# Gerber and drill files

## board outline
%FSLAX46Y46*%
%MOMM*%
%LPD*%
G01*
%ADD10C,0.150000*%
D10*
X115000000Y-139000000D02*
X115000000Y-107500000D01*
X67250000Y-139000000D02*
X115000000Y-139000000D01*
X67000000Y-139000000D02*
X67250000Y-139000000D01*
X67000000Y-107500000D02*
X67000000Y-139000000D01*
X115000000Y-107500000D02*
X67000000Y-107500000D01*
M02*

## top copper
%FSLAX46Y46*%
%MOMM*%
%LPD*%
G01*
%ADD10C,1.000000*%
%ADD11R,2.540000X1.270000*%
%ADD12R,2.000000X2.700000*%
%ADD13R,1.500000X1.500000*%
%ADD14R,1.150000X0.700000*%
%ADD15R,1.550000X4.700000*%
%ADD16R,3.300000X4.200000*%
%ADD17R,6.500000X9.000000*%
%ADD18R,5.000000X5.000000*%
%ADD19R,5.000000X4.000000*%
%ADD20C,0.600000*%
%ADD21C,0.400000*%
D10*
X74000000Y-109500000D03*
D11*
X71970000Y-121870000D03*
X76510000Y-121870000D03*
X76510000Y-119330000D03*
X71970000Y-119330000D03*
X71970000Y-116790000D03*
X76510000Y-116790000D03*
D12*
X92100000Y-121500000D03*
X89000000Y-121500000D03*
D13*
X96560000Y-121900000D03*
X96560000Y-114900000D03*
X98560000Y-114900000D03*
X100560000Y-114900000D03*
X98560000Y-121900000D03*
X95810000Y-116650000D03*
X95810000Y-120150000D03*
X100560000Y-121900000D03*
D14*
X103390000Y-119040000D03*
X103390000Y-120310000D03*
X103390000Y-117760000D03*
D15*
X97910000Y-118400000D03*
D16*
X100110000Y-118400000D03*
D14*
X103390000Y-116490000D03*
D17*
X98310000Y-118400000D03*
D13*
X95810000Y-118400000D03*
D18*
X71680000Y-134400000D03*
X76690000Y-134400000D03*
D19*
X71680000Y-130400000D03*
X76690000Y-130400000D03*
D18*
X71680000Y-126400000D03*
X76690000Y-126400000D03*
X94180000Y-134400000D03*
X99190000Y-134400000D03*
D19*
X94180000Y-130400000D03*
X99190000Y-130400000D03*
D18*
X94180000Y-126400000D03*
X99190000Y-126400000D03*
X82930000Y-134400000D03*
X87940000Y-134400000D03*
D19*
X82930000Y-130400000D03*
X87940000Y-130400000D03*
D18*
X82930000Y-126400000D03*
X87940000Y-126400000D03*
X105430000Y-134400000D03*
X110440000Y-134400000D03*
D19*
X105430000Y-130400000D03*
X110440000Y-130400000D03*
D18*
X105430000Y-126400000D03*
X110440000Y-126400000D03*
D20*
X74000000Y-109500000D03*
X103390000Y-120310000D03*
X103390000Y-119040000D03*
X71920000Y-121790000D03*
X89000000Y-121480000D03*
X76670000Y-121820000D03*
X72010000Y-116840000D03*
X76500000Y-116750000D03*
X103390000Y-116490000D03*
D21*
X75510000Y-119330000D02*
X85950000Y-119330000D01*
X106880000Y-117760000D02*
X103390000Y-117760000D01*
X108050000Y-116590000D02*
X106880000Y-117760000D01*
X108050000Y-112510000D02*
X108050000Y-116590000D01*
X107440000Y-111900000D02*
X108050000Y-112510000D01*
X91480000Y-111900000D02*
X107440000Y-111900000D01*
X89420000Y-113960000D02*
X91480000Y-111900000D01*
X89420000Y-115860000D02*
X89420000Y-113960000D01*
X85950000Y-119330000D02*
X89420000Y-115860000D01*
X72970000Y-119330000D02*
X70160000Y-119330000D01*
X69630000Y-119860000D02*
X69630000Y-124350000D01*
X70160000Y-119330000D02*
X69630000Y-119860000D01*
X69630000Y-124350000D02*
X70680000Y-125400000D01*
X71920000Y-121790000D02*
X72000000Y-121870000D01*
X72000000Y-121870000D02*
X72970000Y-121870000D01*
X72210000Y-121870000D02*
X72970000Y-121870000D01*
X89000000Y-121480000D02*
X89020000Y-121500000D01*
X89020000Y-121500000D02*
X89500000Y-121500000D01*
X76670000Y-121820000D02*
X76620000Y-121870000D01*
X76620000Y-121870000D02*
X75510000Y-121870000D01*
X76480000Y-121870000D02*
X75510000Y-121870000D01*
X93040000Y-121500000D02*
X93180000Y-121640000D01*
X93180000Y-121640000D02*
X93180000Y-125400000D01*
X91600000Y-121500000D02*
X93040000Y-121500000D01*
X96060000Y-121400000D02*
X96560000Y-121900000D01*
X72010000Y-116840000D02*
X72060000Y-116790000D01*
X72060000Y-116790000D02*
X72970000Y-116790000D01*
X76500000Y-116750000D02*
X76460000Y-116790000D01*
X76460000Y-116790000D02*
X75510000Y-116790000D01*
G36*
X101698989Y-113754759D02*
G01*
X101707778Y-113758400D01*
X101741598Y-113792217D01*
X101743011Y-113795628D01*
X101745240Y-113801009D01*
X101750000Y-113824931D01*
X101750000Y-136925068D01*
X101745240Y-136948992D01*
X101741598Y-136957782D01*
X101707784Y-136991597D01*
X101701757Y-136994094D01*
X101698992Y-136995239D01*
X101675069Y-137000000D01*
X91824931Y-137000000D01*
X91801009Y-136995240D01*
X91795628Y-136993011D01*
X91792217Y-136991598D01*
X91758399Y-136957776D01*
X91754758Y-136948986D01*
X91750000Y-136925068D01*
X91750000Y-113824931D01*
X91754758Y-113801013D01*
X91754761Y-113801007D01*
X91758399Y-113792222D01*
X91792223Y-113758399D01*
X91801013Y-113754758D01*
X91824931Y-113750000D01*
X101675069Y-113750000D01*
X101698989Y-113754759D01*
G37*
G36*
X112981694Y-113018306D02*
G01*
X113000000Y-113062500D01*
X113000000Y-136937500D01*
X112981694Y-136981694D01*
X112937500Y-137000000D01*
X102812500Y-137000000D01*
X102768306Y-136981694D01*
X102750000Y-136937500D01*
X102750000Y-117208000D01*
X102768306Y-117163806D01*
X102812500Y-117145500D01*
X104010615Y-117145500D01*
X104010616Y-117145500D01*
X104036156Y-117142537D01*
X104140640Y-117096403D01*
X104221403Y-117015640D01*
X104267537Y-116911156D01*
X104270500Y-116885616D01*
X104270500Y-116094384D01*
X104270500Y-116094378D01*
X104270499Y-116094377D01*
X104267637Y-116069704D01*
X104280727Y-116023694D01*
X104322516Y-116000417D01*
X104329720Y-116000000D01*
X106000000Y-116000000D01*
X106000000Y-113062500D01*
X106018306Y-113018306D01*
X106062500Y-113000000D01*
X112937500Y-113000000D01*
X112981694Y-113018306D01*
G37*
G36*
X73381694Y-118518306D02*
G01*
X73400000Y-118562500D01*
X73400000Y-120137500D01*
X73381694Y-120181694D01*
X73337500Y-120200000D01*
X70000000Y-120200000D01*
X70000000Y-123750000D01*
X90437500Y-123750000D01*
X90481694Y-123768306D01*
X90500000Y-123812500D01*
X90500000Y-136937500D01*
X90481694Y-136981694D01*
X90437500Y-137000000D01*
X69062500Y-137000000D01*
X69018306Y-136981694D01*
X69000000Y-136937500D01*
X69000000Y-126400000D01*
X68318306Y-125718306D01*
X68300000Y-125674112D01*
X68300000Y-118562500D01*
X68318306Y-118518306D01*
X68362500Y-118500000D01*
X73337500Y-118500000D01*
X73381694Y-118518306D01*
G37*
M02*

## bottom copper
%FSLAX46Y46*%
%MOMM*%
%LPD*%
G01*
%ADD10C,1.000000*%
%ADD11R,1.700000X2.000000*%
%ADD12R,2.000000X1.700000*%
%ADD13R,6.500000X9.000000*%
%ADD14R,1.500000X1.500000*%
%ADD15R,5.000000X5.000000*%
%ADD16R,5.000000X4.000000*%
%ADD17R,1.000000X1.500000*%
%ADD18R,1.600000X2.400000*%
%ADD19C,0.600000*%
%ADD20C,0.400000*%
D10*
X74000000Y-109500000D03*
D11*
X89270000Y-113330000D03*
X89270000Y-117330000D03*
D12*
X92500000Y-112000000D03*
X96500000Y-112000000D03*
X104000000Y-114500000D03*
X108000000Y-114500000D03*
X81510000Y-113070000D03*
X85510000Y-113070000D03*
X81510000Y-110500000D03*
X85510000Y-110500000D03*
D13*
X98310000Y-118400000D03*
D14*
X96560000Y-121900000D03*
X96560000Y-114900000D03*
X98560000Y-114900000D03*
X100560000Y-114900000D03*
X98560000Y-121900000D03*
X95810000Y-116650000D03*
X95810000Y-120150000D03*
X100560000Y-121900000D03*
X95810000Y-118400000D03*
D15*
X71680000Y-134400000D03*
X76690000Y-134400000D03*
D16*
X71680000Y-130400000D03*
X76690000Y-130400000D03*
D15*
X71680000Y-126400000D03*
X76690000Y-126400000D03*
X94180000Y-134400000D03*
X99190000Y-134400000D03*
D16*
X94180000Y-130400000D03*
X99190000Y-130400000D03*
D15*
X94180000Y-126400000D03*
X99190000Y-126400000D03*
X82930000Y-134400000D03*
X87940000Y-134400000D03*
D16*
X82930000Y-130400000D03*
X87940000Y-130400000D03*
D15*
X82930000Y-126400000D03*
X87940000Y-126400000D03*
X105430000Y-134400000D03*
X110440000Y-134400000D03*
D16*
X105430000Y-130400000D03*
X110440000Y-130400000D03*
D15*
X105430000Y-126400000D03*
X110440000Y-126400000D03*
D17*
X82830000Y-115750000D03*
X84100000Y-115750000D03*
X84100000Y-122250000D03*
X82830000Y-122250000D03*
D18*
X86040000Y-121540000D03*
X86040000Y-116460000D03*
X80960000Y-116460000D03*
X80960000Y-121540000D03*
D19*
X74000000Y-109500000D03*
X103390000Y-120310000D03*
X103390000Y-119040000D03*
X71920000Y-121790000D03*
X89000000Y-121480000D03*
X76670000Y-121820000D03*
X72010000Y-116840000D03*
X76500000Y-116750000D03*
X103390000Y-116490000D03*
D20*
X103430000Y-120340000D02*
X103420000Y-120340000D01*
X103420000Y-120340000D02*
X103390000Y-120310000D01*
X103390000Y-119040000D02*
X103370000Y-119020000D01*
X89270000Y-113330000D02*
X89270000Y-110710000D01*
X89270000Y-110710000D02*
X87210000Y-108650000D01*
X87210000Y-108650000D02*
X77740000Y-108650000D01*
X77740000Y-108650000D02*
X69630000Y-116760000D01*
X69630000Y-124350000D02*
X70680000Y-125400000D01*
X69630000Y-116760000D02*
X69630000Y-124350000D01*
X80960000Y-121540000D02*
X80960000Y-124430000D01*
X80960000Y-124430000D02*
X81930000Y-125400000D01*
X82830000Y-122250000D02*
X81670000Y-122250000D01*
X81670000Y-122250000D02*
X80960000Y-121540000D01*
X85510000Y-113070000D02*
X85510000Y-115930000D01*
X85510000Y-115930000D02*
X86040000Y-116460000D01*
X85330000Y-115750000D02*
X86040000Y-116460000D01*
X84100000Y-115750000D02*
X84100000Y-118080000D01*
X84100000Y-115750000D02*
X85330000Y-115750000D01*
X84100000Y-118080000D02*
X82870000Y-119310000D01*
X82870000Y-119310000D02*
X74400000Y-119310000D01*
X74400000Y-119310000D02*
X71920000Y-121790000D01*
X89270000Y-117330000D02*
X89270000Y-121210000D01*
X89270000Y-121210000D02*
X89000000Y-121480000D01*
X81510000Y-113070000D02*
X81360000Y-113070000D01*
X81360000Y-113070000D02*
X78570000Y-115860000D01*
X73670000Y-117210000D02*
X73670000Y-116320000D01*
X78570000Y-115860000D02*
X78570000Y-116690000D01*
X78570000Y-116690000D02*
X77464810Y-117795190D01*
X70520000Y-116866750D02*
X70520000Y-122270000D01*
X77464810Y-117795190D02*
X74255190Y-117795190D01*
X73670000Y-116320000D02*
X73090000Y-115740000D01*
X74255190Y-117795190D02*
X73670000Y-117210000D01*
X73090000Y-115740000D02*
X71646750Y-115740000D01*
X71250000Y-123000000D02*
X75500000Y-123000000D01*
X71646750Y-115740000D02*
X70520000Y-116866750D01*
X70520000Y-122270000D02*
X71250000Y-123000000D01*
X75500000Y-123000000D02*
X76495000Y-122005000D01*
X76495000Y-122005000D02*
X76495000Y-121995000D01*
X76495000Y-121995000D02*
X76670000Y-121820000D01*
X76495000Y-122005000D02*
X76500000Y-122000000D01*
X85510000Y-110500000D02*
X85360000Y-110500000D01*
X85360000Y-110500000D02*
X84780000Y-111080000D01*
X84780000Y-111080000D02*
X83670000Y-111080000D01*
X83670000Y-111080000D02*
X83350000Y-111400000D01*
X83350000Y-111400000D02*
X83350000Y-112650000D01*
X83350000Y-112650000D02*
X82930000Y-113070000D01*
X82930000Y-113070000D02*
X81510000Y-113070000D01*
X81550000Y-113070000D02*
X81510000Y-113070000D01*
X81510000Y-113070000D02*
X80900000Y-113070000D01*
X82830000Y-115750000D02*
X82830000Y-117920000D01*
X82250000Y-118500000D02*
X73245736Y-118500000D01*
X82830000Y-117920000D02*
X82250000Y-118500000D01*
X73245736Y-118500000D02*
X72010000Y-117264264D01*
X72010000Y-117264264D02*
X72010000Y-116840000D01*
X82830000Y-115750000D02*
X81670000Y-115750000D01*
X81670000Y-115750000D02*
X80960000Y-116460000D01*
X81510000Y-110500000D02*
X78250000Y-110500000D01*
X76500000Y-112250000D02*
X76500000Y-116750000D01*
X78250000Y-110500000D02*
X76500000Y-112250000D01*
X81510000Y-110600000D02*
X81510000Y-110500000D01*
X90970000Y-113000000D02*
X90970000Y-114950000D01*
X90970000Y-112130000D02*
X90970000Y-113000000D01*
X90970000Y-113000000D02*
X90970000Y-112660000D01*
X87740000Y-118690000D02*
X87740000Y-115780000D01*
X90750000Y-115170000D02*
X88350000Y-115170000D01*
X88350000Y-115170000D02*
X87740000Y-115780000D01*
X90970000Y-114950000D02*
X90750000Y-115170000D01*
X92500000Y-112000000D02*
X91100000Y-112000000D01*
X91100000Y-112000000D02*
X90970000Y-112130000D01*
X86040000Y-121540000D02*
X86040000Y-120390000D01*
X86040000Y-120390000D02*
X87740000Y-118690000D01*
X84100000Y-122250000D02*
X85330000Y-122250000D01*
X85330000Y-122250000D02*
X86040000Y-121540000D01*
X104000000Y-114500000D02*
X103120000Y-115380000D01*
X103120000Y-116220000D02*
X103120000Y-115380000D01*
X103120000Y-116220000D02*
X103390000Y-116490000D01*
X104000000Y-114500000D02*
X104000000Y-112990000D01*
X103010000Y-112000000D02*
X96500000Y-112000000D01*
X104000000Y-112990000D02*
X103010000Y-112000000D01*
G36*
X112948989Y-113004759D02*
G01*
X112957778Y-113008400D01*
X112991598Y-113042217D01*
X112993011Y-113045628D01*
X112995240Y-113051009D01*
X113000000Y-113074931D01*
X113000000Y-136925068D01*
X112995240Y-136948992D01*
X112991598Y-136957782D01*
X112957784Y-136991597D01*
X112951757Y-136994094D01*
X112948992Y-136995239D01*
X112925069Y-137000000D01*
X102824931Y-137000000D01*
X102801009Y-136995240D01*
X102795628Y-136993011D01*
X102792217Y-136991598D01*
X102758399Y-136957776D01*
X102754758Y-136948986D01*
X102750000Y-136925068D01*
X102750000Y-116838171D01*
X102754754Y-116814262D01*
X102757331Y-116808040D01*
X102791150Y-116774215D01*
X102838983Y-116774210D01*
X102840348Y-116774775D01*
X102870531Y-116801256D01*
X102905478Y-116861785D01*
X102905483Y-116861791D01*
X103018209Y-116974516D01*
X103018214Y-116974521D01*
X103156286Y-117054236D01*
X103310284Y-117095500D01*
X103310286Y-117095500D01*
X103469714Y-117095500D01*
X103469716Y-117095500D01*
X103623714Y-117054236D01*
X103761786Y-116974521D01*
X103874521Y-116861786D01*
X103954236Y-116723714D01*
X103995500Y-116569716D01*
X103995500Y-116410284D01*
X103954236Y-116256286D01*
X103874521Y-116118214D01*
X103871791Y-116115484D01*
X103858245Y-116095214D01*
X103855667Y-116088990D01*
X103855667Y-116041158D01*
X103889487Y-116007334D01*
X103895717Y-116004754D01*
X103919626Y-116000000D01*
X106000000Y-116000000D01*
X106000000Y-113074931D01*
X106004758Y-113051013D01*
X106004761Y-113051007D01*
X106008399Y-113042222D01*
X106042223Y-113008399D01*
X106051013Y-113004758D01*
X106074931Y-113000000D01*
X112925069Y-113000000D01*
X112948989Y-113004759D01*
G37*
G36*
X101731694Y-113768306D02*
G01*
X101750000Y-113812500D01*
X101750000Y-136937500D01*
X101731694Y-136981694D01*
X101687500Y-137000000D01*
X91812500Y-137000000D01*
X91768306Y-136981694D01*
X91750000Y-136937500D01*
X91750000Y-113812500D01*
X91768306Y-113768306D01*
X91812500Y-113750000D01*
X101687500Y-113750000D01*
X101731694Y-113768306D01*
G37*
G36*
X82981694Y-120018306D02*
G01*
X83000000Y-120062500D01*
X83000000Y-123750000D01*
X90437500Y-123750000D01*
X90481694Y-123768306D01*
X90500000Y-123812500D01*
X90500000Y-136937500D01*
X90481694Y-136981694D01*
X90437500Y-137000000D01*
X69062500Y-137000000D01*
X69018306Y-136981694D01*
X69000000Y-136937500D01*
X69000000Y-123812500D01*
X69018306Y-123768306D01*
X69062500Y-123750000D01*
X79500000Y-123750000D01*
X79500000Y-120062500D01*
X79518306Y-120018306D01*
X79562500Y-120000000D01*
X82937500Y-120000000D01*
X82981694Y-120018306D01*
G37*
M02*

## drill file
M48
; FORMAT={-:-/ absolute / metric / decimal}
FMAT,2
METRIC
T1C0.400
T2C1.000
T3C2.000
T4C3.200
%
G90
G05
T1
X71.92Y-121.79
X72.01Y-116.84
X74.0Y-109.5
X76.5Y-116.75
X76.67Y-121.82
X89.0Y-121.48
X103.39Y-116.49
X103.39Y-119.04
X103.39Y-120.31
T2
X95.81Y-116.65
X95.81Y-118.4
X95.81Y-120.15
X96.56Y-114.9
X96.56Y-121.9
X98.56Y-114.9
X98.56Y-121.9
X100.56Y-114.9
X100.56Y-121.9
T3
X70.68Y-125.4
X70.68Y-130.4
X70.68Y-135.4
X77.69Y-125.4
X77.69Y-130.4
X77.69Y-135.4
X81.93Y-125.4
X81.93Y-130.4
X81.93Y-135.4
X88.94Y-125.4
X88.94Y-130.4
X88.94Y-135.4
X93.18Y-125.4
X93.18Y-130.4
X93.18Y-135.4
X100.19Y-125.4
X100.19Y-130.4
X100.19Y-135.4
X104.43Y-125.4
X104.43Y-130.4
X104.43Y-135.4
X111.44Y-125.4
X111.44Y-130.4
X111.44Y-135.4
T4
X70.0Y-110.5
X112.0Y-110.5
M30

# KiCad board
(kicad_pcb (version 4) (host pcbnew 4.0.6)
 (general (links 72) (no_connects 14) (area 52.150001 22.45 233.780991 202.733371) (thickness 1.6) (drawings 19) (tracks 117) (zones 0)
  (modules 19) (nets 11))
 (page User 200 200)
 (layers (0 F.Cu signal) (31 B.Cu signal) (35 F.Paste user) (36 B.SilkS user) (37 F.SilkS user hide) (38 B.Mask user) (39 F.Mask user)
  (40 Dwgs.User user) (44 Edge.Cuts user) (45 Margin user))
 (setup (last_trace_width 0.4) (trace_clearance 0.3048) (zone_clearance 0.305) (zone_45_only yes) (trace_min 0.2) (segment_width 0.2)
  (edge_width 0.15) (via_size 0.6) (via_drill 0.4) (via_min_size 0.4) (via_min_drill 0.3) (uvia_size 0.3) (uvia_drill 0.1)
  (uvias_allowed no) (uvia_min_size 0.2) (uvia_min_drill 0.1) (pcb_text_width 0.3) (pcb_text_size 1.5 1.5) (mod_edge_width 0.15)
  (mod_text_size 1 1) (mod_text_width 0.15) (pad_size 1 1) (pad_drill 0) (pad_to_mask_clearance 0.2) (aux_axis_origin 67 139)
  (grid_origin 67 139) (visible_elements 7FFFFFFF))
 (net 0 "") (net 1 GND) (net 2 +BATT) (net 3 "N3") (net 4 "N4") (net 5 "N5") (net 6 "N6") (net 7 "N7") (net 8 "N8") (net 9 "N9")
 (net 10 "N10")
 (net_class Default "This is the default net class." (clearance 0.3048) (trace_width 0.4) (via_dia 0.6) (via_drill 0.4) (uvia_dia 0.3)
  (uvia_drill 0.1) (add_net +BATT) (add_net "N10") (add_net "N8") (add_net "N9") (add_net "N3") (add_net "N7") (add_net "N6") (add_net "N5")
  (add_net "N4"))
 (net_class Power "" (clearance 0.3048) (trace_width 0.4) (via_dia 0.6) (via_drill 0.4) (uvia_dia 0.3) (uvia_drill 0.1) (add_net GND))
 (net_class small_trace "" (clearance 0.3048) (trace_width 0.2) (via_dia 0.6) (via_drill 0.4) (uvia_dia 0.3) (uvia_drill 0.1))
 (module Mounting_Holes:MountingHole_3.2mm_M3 (layer F.Cu) (at 112 110.5)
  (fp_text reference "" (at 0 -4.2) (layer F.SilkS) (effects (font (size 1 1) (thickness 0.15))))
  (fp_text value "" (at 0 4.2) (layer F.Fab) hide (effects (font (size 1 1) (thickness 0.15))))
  (pad 1 np_thru_hole circle (at 0 0) (size 3.2 3.2) (drill 3.2) (layers *.Cu *.Mask)))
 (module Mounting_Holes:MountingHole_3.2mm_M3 (layer F.Cu) (at 70 110.5)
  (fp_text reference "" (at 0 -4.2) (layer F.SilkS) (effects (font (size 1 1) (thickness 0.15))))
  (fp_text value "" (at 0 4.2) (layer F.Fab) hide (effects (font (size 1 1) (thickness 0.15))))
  (pad 1 np_thru_hole circle (at 0 0) (size 3.2 3.2) (drill 3.2) (layers *.Cu *.Mask)))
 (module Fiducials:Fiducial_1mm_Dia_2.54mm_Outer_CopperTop (layer B.Cu) (at 74 109.5)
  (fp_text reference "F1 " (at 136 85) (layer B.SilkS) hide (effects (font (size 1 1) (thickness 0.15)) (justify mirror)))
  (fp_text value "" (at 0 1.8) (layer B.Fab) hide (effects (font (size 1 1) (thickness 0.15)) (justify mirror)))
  (pad 2 smd circle (at 0 0) (size 1 1) (layers B.Cu B.Mask) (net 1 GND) (solder_mask_margin 0.77) (clearance 0.77)))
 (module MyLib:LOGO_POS (layer F.Cu) (at 84 115)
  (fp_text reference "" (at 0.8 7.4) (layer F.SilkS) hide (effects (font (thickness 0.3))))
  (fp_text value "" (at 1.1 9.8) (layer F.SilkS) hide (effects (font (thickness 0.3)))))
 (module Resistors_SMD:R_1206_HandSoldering (layer B.Cu) (at 89.27 115.33 270)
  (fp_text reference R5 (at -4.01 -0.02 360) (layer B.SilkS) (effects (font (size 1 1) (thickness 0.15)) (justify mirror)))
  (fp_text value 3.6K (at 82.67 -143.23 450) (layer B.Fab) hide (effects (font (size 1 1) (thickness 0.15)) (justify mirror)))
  (pad 1 smd rect (at -2 0 270) (size 2 1.7) (layers B.Cu B.Mask) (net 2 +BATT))
  (pad 2 smd rect (at 2 0 270) (size 2 1.7) (layers B.Cu B.Mask) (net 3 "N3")))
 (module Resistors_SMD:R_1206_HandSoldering (layer B.Cu) (at 94.5 112)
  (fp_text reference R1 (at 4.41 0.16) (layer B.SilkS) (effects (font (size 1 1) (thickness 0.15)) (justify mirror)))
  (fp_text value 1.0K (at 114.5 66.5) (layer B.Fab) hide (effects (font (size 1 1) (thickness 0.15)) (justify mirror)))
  (pad 1 smd rect (at -2 0) (size 2 1.7) (layers B.Cu B.Mask) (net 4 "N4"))
  (pad 2 smd rect (at 2 0) (size 2 1.7) (layers B.Cu B.Mask) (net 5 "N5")))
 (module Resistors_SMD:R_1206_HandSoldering (layer B.Cu) (at 106 114.5)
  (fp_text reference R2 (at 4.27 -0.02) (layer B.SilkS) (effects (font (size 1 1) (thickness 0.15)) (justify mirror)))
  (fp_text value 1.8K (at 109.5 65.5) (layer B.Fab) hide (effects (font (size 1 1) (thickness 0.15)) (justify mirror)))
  (pad 1 smd rect (at -2 0) (size 2 1.7) (layers B.Cu B.Mask) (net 5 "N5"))
  (pad 2 smd rect (at 2 0) (size 2 1.7) (layers B.Cu B.Mask) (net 1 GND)))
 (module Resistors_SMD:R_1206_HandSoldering (layer B.Cu) (at 83.51 113.07)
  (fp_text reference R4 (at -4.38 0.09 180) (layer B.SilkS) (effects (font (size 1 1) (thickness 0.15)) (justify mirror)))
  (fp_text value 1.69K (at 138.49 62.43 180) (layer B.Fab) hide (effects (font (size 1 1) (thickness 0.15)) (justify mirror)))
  (pad 1 smd rect (at -2 0) (size 2 1.7) (layers B.Cu B.Mask) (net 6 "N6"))
  (pad 2 smd rect (at 2 0) (size 2 1.7) (layers B.Cu B.Mask) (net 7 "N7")))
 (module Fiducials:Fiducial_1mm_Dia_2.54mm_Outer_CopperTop (layer F.Cu) (at 74 109.5)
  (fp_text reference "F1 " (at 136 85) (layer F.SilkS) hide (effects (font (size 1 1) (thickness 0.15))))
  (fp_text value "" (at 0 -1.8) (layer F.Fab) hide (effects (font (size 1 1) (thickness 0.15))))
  (pad 1 smd circle (at 0 0) (size 1 1) (layers F.Cu F.Mask) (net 1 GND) (solder_mask_margin 0.77) (clearance 0.77)))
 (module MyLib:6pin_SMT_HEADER (layer F.Cu) (at 74.24 119.33 270)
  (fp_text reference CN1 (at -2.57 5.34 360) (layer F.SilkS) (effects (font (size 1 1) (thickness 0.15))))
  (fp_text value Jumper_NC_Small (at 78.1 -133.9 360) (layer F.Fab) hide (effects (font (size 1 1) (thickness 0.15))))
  (pad 5 smd rect (at 2.54 1.27 270) (size 1.27 2.54) (drill (offset 0 1)) (layers F.Cu F.Paste F.Mask) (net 7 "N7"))
  (pad 6 smd rect (at 2.54 -1.27 270) (size 1.27 2.54) (drill (offset 0 -1)) (layers F.Cu F.Paste F.Mask) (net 6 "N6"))
  (pad 4 smd rect (at 0 -1.27 270) (size 1.27 2.54) (drill (offset 0 -1)) (layers F.Cu F.Paste F.Mask) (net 1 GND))
  (pad 3 smd rect (at 0 1.27 270) (size 1.27 2.54) (drill (offset 0 1)) (layers F.Cu F.Paste F.Mask) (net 2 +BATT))
  (pad 1 smd rect (at -2.54 1.27 270) (size 1.27 2.54) (drill (offset 0 1)) (layers F.Cu F.Paste F.Mask) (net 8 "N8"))
  (pad 2 smd rect (at -2.54 -1.27 270) (size 1.27 2.54) (drill (offset 0 -1)) (layers F.Cu F.Paste F.Mask) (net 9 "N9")))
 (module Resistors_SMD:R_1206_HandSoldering (layer B.Cu) (at 83.51 110.5)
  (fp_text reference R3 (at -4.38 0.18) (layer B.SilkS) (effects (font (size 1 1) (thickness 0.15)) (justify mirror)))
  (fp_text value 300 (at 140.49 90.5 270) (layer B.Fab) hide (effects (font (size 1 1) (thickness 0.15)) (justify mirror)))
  (pad 1 smd rect (at -2 0) (size 2 1.7) (layers B.Cu B.Mask) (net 9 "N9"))
  (pad 2 smd rect (at 2 0) (size 2 1.7) (layers B.Cu B.Mask) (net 6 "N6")))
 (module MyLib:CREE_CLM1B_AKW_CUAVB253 (layer F.Cu) (at 90.5 121.5)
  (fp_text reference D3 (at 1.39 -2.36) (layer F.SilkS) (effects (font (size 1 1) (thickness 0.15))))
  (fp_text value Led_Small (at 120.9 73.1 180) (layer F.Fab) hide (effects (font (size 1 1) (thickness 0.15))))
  (pad 1 smd rect (at 1.1 0) (size 2 2.7) (drill (offset 0.5 0)) (layers F.Cu F.Paste F.Mask) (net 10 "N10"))
  (pad 2 smd rect (at -1 0) (size 2 2.7) (drill (offset -0.5 0)) (layers F.Cu F.Paste F.Mask) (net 3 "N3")))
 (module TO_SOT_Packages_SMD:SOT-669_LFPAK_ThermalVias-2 (layer F.Cu) (at 99.6 118.4 180)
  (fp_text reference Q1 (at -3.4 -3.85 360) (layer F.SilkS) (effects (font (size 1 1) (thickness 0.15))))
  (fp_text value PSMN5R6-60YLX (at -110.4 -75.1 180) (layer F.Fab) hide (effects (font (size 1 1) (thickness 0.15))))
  (pad 5 smd rect (at 1.29 0 90) (size 9 6.5) (layers *.Mask B.Cu) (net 10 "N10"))
  (pad 5 thru_hole rect (at 3.04 -3.5 90) (size 1.5 1.5) (drill 1) (layers *.Cu *.Mask) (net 10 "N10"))
  (pad 5 thru_hole rect (at 3.04 3.5 90) (size 1.5 1.5) (drill 1) (layers *.Cu *.Mask) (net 10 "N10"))
  (pad 5 thru_hole rect (at 1.04 3.5 90) (size 1.5 1.5) (drill 1) (layers *.Cu B.SilkS F.Mask) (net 10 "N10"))
  (pad 5 thru_hole rect (at -0.96 3.5 90) (size 1.5 1.5) (drill 1) (layers *.Cu B.SilkS F.Mask) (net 10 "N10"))
  (pad 5 thru_hole rect (at 1.04 -3.5 90) (size 1.5 1.5) (drill 1) (layers *.Cu *.Mask) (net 10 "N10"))
  (pad 5 thru_hole rect (at 3.79 1.75 90) (size 1.5 1.5) (drill 1) (layers *.Cu *.Mask) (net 10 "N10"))
  (pad 5 thru_hole rect (at 3.79 -1.75 90) (size 1.5 1.5) (drill 1) (layers *.Cu *.Mask) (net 10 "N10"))
  (pad 5 thru_hole rect (at -0.96 -3.5 90) (size 1.5 1.5) (drill 1) (layers *.Cu *.Mask) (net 10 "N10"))
  (pad 5 smd rect (at -0.76 -1.15 180) (size 0.6 0.9) (layers F.Paste) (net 10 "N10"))
  (pad 5 smd rect (at -1.61 -1.15 180) (size 0.6 0.9) (layers F.Paste) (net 10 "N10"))
  (pad 5 smd rect (at 0.09 -1.15 180) (size 0.6 0.9) (layers F.Paste) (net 10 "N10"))
  (pad 5 smd rect (at -0.76 1.15 180) (size 0.6 0.9) (layers F.Paste) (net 10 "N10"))
  (pad 5 smd rect (at -1.61 1.15 180) (size 0.6 0.9) (layers F.Paste) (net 10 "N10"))
  (pad 5 smd rect (at 0.09 1.15 180) (size 0.6 0.9) (layers F.Paste) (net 10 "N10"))
  (pad 5 smd rect (at 0.09 0 180) (size 0.6 0.9) (layers F.Paste) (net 10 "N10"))
  (pad 5 smd rect (at -1.61 0 180) (size 0.6 0.9) (layers F.Paste) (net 10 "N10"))
  (pad 5 smd rect (at 1.94 -1.88 90) (size 0.6 0.9) (layers F.Paste) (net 10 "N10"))
  (pad 5 smd rect (at 1.94 1.88 90) (size 0.6 0.9) (layers F.Paste) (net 10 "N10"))
  (pad 5 smd rect (at 1.94 -0.6 90) (size 0.6 0.9) (layers F.Paste) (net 10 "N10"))
  (pad 2 smd rect (at -3.79 -0.64 90) (size 0.7 1.15) (layers F.Cu F.Paste F.Mask) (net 1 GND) (solder_mask_margin 0.07)
   (solder_paste_margin -0.05))
  (pad 1 smd rect (at -3.79 -1.91 90) (size 0.7 1.15) (layers F.Cu F.Paste F.Mask) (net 1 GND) (solder_mask_margin 0.07)
   (solder_paste_margin -0.05))
  (pad 3 smd rect (at -3.79 0.64 90) (size 0.7 1.15) (layers F.Cu F.Paste F.Mask) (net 1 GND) (solder_mask_margin 0.07)
   (solder_paste_margin -0.05))
  (pad 5 smd rect (at 1.69 0 90) (size 4.7 1.55) (layers F.Cu F.Mask) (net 10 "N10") (solder_mask_margin 0.07))
  (pad 5 smd rect (at -0.51 0 90) (size 4.2 3.3) (layers F.Cu F.Mask) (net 10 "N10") (solder_mask_margin 0.07))
  (pad 4 smd rect (at -3.79 1.91 90) (size 0.7 1.15) (layers F.Cu F.Paste F.Mask) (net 5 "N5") (solder_mask_margin 0.07)
   (solder_paste_margin -0.05))
  (pad 5 smd rect (at 1.94 0.6 90) (size 0.6 0.9) (layers F.Paste) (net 10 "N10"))
  (pad 5 smd rect (at -0.76 0 180) (size 0.6 0.9) (layers F.Paste) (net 10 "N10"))
  (pad 5 smd rect (at 1.29 0 90) (size 9 6.5) (layers *.Mask F.Cu) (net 10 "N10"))
  (pad 5 thru_hole rect (at 3.79 0 90) (size 1.5 1.5) (drill 1) (layers *.Cu *.Mask) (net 10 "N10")))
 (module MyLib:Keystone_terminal (layer F.Cu) (at 74.1 130.4 90)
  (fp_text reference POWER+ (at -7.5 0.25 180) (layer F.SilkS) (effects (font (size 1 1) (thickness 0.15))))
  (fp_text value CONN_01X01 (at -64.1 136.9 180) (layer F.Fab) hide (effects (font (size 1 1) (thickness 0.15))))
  (pad 1 thru_hole rect (at -5 -3.42 90) (size 5 5) (drill 2 (offset 1 1)) (layers *.Cu *.Mask F.Paste) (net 2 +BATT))
  (pad 1 thru_hole rect (at -5 3.59 90) (size 5 5) (drill 2 (offset 1 -1)) (layers *.Cu *.Mask F.Paste) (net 2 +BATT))
  (pad 1 thru_hole rect (at 0 -3.42 90) (size 4 5) (drill 2 (offset 0 1)) (layers *.Cu *.Mask F.Paste) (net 2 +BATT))
  (pad 1 thru_hole rect (at 0 3.59 90) (size 4 5) (drill 2 (offset 0 -1)) (layers *.Cu *.Mask F.Paste) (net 2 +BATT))
  (pad 1 thru_hole rect (at 5 -3.42 90) (size 5 5) (drill 2 (offset -1 1)) (layers *.Cu *.Mask F.Paste) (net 2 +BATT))
  (pad 1 thru_hole rect (at 5 3.59 90) (size 5 5) (drill 2 (offset -1 -1)) (layers *.Cu *.Mask F.Paste) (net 2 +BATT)))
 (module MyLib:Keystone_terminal (layer F.Cu) (at 96.6 130.4 90)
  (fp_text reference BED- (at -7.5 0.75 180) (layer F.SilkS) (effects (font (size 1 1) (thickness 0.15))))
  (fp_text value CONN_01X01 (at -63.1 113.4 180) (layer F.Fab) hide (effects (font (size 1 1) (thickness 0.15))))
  (pad 1 thru_hole rect (at -5 -3.42 90) (size 5 5) (drill 2 (offset 1 1)) (layers *.Cu *.Mask F.Paste) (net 10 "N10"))
  (pad 1 thru_hole rect (at -5 3.59 90) (size 5 5) (drill 2 (offset 1 -1)) (layers *.Cu *.Mask F.Paste) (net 10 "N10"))
  (pad 1 thru_hole rect (at 0 -3.42 90) (size 4 5) (drill 2 (offset 0 1)) (layers *.Cu *.Mask F.Paste) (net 10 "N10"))
  (pad 1 thru_hole rect (at 0 3.59 90) (size 4 5) (drill 2 (offset 0 -1)) (layers *.Cu *.Mask F.Paste) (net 10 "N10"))
  (pad 1 thru_hole rect (at 5 -3.42 90) (size 5 5) (drill 2 (offset -1 1)) (layers *.Cu *.Mask F.Paste) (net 10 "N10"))
  (pad 1 thru_hole rect (at 5 3.59 90) (size 5 5) (drill 2 (offset -1 -1)) (layers *.Cu *.Mask F.Paste) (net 10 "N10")))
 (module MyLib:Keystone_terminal (layer F.Cu) (at 85.35 130.4 90)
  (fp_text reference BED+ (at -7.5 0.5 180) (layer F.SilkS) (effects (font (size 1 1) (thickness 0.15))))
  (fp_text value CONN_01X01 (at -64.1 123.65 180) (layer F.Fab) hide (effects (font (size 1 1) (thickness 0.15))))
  (pad 1 thru_hole rect (at -5 -3.42 90) (size 5 5) (drill 2 (offset 1 1)) (layers *.Cu *.Mask F.Paste) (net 2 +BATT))
  (pad 1 thru_hole rect (at -5 3.59 90) (size 5 5) (drill 2 (offset 1 -1)) (layers *.Cu *.Mask F.Paste) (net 2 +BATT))
  (pad 1 thru_hole rect (at 0 -3.42 90) (size 4 5) (drill 2 (offset 0 1)) (layers *.Cu *.Mask F.Paste) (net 2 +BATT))
  (pad 1 thru_hole rect (at 0 3.59 90) (size 4 5) (drill 2 (offset 0 -1)) (layers *.Cu *.Mask F.Paste) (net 2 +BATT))
  (pad 1 thru_hole rect (at 5 -3.42 90) (size 5 5) (drill 2 (offset -1 1)) (layers *.Cu *.Mask F.Paste) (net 2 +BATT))
  (pad 1 thru_hole rect (at 5 3.59 90) (size 5 5) (drill 2 (offset -1 -1)) (layers *.Cu *.Mask F.Paste) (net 2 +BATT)))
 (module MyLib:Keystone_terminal (layer F.Cu) (at 107.85 130.4 90)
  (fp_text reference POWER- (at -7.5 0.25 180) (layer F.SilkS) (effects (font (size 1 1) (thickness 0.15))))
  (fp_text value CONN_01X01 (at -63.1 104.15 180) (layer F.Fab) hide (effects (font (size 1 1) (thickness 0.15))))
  (pad 1 thru_hole rect (at -5 -3.42 90) (size 5 5) (drill 2 (offset 1 1)) (layers *.Cu *.Mask F.Paste) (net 1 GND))
  (pad 1 thru_hole rect (at -5 3.59 90) (size 5 5) (drill 2 (offset 1 -1)) (layers *.Cu *.Mask F.Paste) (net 1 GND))
  (pad 1 thru_hole rect (at 0 -3.42 90) (size 4 5) (drill 2 (offset 0 1)) (layers *.Cu *.Mask F.Paste) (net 1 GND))
  (pad 1 thru_hole rect (at 0 3.59 90) (size 4 5) (drill 2 (offset 0 -1)) (layers *.Cu *.Mask F.Paste) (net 1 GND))
  (pad 1 thru_hole rect (at 5 -3.42 90) (size 5 5) (drill 2 (offset -1 1)) (layers *.Cu *.Mask F.Paste) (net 1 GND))
  (pad 1 thru_hole rect (at 5 3.59 90) (size 5 5) (drill 2 (offset -1 -1)) (layers *.Cu *.Mask F.Paste) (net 1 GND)))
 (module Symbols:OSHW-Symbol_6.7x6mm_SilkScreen (layer F.Cu) (at 108.5 119)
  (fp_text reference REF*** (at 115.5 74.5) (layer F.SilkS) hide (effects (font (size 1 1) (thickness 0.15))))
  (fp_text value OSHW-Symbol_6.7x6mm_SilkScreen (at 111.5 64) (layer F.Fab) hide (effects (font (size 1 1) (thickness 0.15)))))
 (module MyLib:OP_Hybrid (layer B.Cu) (at 83.5 119 270)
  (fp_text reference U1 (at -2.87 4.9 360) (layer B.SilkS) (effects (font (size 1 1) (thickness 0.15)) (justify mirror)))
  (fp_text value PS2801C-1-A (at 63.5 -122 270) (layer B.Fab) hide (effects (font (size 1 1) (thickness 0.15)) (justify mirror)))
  (pad 1 smd rect (at -3.25 0.67) (size 1 1.5) (layers B.Cu B.Mask) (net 8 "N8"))
  (pad 3 smd rect (at -3.25 -0.6) (size 1 1.5) (layers B.Cu B.Mask) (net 7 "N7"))
  (pad 4 smd rect (at 3.25 -0.6) (size 1 1.5) (layers B.Cu B.Mask) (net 4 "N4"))
  (pad 6 smd rect (at 3.25 0.67) (size 1 1.5) (layers B.Cu B.Mask) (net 2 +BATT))
  (pad 4 smd rect (at 2.54 -2.54 270) (size 2.4 1.6) (layers B.Cu B.Mask) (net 4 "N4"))
  (pad 3 smd rect (at -2.54 -2.54 270) (size 2.4 1.6) (layers B.Cu B.Mask) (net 7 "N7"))
  (pad 1 smd rect (at -2.54 2.54 270) (size 2.4 1.6) (layers B.Cu B.Mask) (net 8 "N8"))
  (pad 6 smd rect (at 2.54 2.54 270) (size 2.4 1.6) (layers B.Cu B.Mask) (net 2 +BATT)))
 (gr_line (start 115 139) (end 115 107.5) (angle 90) (layer Edge.Cuts) (width 0.15))
 (gr_line (start 67.25 139) (end 115 139) (angle 90) (layer Edge.Cuts) (width 0.15))
 (gr_line (start 67 139) (end 67.25 139) (angle 90) (layer Edge.Cuts) (width 0.15))
 (gr_line (start 67 107.5) (end 67 139) (angle 90) (layer Edge.Cuts) (width 0.15))
 (gr_line (start 115 107.5) (end 67 107.5) (angle 90) (layer Edge.Cuts) (width 0.15))
 (segment (start 75.51 119.33) (end 85.95 119.33) (width 0.4) (layer F.Cu) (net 1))
 (segment (start 106.88 117.76) (end 103.39 117.76) (width 0.4) (layer F.Cu) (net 1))
 (segment (start 108.05 116.59) (end 106.88 117.76) (width 0.4) (layer F.Cu) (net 1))
 (segment (start 108.05 112.51) (end 108.05 116.59) (width 0.4) (layer F.Cu) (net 1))
 (segment (start 107.44 111.9) (end 108.05 112.51) (width 0.4) (layer F.Cu) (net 1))
 (segment (start 91.48 111.9) (end 107.44 111.9) (width 0.4) (layer F.Cu) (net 1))
 (segment (start 89.42 113.96) (end 91.48 111.9) (width 0.4) (layer F.Cu) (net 1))
 (segment (start 89.42 115.86) (end 89.42 113.96) (width 0.4) (layer F.Cu) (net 1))
 (segment (start 85.95 119.33) (end 89.42 115.86) (width 0.4) (layer F.Cu) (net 1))
 (via (at 74 109.5) (size 0.6) (drill 0.4) (layers F.Cu B.Cu) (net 1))
 (via (at 103.39 120.31) (size 0.6) (drill 0.4) (layers F.Cu B.Cu) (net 1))
 (segment (start 103.43 120.34) (end 103.42 120.34) (width 0.4) (layer B.Cu) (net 1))
 (segment (start 103.42 120.34) (end 103.39 120.31) (width 0.4) (layer B.Cu) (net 1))
 (via (at 103.39 119.04) (size 0.6) (drill 0.4) (layers F.Cu B.Cu) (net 1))
 (segment (start 103.39 119.04) (end 103.37 119.02) (width 0.4) (layer B.Cu) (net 1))
 (segment (start 89.27 113.33) (end 89.27 110.71) (width 0.4) (layer B.Cu) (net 2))
 (segment (start 89.27 110.71) (end 87.21 108.65) (width 0.4) (layer B.Cu) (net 2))
 (segment (start 87.21 108.65) (end 77.74 108.65) (width 0.4) (layer B.Cu) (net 2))
 (segment (start 77.74 108.65) (end 69.63 116.76) (width 0.4) (layer B.Cu) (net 2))
 (segment (start 69.63 124.35) (end 70.68 125.4) (width 0.4) (layer B.Cu) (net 2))
 (segment (start 69.63 116.76) (end 69.63 124.35) (width 0.4) (layer B.Cu) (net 2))
 (segment (start 72.97 119.33) (end 70.16 119.33) (width 0.4) (layer F.Cu) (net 2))
 (segment (start 69.63 119.86) (end 69.63 124.35) (width 0.4) (layer F.Cu) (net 2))
 (segment (start 70.16 119.33) (end 69.63 119.86) (width 0.4) (layer F.Cu) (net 2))
 (segment (start 69.63 124.35) (end 70.68 125.4) (width 0.4) (layer F.Cu) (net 2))
 (segment (start 80.96 121.54) (end 80.96 124.43) (width 0.4) (layer B.Cu) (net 2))
 (segment (start 80.96 124.43) (end 81.93 125.4) (width 0.4) (layer B.Cu) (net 2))
 (segment (start 82.83 122.25) (end 81.67 122.25) (width 0.4) (layer B.Cu) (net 2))
 (segment (start 81.67 122.25) (end 80.96 121.54) (width 0.4) (layer B.Cu) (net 2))
 (segment (start 85.51 113.07) (end 85.51 115.93) (width 0.4) (layer B.Cu) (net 7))
 (segment (start 85.51 115.93) (end 86.04 116.46) (width 0.4) (layer B.Cu) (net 7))
 (segment (start 85.33 115.75) (end 86.04 116.46) (width 0.4) (layer B.Cu) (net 7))
 (segment (start 84.1 115.75) (end 84.1 118.08) (width 0.4) (layer B.Cu) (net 7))
 (segment (start 84.1 115.75) (end 85.33 115.75) (width 0.4) (layer B.Cu) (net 7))
 (segment (start 84.1 118.08) (end 82.87 119.31) (width 0.4) (layer B.Cu) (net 7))
 (segment (start 82.87 119.31) (end 74.4 119.31) (width 0.4) (layer B.Cu) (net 7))
 (segment (start 74.4 119.31) (end 71.92 121.79) (width 0.4) (layer B.Cu) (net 7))
 (segment (start 71.92 121.79) (end 72 121.87) (width 0.4) (layer F.Cu) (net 7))
 (via (at 71.92 121.79) (size 0.6) (drill 0.4) (layers F.Cu B.Cu) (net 7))
 (segment (start 72 121.87) (end 72.97 121.87) (width 0.4) (layer F.Cu) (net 7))
 (segment (start 72.21 121.87) (end 72.97 121.87) (width 0.4) (layer F.Cu) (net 7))
 (segment (start 89.27 117.33) (end 89.27 121.21) (width 0.4) (layer B.Cu) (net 3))
 (segment (start 89 121.48) (end 89.02 121.5) (width 0.4) (layer F.Cu) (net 3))
 (via (at 89 121.48) (size 0.6) (drill 0.4) (layers F.Cu B.Cu) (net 3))
 (segment (start 89.27 121.21) (end 89 121.48) (width 0.4) (layer B.Cu) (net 3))
 (segment (start 89.02 121.5) (end 89.5 121.5) (width 0.4) (layer F.Cu) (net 3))
 (segment (start 81.51 113.07) (end 81.36 113.07) (width 0.4) (layer B.Cu) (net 6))
 (segment (start 81.36 113.07) (end 78.57 115.86) (width 0.4) (layer B.Cu) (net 6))
 (segment (start 73.67 117.21) (end 73.67 116.32) (width 0.4) (layer B.Cu) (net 6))
 (segment (start 78.57 115.86) (end 78.57 116.69) (width 0.4) (layer B.Cu) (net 6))
 (segment (start 78.57 116.69) (end 77.46481 117.79519) (width 0.4) (layer B.Cu) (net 6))
 (segment (start 70.52 116.86675) (end 70.52 122.27) (width 0.4) (layer B.Cu) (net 6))
 (segment (start 77.46481 117.79519) (end 74.25519 117.79519) (width 0.4) (layer B.Cu) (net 6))
 (segment (start 73.67 116.32) (end 73.09 115.74) (width 0.4) (layer B.Cu) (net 6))
 (segment (start 74.25519 117.79519) (end 73.67 117.21) (width 0.4) (layer B.Cu) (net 6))
 (segment (start 73.09 115.74) (end 71.64675 115.74) (width 0.4) (layer B.Cu) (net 6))
 (segment (start 71.25 123) (end 75.5 123) (width 0.4) (layer B.Cu) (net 6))
 (segment (start 71.64675 115.74) (end 70.52 116.86675) (width 0.4) (layer B.Cu) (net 6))
 (segment (start 70.52 122.27) (end 71.25 123) (width 0.4) (layer B.Cu) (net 6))
 (segment (start 75.5 123) (end 76.495 122.005) (width 0.4) (layer B.Cu) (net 6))
 (segment (start 76.495 122.005) (end 76.495 121.995) (width 0.4) (layer B.Cu) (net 6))
 (segment (start 76.67 121.82) (end 76.62 121.87) (width 0.4) (layer F.Cu) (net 6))
 (via (at 76.67 121.82) (size 0.6) (drill 0.4) (layers F.Cu B.Cu) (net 6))
 (segment (start 76.495 121.995) (end 76.67 121.82) (width 0.4) (layer B.Cu) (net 6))
 (segment (start 76.62 121.87) (end 75.51 121.87) (width 0.4) (layer F.Cu) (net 6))
 (segment (start 76.495 122.005) (end 76.5 122) (width 0.4) (layer B.Cu) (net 6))
 (segment (start 85.51 110.5) (end 85.36 110.5) (width 0.4) (layer B.Cu) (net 6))
 (segment (start 85.36 110.5) (end 84.78 111.08) (width 0.4) (layer B.Cu) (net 6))
 (segment (start 84.78 111.08) (end 83.67 111.08) (width 0.4) (layer B.Cu) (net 6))
 (segment (start 83.67 111.08) (end 83.35 111.4) (width 0.4) (layer B.Cu) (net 6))
 (segment (start 83.35 111.4) (end 83.35 112.65) (width 0.4) (layer B.Cu) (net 6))
 (segment (start 83.35 112.65) (end 82.93 113.07) (width 0.4) (layer B.Cu) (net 6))
 (segment (start 82.93 113.07) (end 81.51 113.07) (width 0.4) (layer B.Cu) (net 6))
 (segment (start 81.55 113.07) (end 81.51 113.07) (width 0.4) (layer B.Cu) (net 6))
 (segment (start 81.51 113.07) (end 80.9 113.07) (width 0.4) (layer B.Cu) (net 6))
 (segment (start 76.48 121.87) (end 75.51 121.87) (width 0.4) (layer F.Cu) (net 6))
 (segment (start 93.04 121.5) (end 93.18 121.64) (width 0.4) (layer F.Cu) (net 10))
 (segment (start 93.18 121.64) (end 93.18 125.4) (width 0.4) (layer F.Cu) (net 10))
 (segment (start 91.6 121.5) (end 93.04 121.5) (width 0.4) (layer F.Cu) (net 10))
 (segment (start 96.06 121.4) (end 96.56 121.9) (width 0.4) (layer F.Cu) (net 10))
 (segment (start 82.83 115.75) (end 82.83 117.92) (width 0.4) (layer B.Cu) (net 8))
 (segment (start 82.25 118.5) (end 73.245736 118.5) (width 0.4) (layer B.Cu) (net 8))
 (segment (start 82.83 117.92) (end 82.25 118.5) (width 0.4) (layer B.Cu) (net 8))
 (segment (start 73.245736 118.5) (end 72.01 117.264264) (width 0.4) (layer B.Cu) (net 8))
 (segment (start 72.01 117.264264) (end 72.01 116.84) (width 0.4) (layer B.Cu) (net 8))
 (segment (start 72.01 116.84) (end 72.06 116.79) (width 0.4) (layer F.Cu) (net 8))
 (via (at 72.01 116.84) (size 0.6) (drill 0.4) (layers F.Cu B.Cu) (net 8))
 (segment (start 72.06 116.79) (end 72.97 116.79) (width 0.4) (layer F.Cu) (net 8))
 (segment (start 82.83 115.75) (end 81.67 115.75) (width 0.4) (layer B.Cu) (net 8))
 (segment (start 81.67 115.75) (end 80.96 116.46) (width 0.4) (layer B.Cu) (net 8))
 (segment (start 81.51 110.5) (end 78.25 110.5) (width 0.4) (layer B.Cu) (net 9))
 (segment (start 76.5 116.75) (end 76.46 116.79) (width 0.4) (layer F.Cu) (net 9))
 (via (at 76.5 116.75) (size 0.6) (drill 0.4) (layers F.Cu B.Cu) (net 9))
 (segment (start 76.5 112.25) (end 76.5 116.75) (width 0.4) (layer B.Cu) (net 9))
 (segment (start 78.25 110.5) (end 76.5 112.25) (width 0.4) (layer B.Cu) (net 9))
 (segment (start 76.46 116.79) (end 75.51 116.79) (width 0.4) (layer F.Cu) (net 9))
 (segment (start 81.51 110.6) (end 81.51 110.5) (width 0.4) (layer B.Cu) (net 9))
 (segment (start 90.97 113) (end 90.97 114.95) (width 0.4) (layer B.Cu) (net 4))
 (segment (start 90.97 112.13) (end 90.97 113) (width 0.4) (layer B.Cu) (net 4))
 (segment (start 90.97 113) (end 90.97 112.66) (width 0.4) (layer B.Cu) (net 4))
 (segment (start 87.74 118.69) (end 87.74 115.78) (width 0.4) (layer B.Cu) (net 4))
 (segment (start 90.75 115.17) (end 88.35 115.17) (width 0.4) (layer B.Cu) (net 4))
 (segment (start 88.35 115.17) (end 87.74 115.78) (width 0.4) (layer B.Cu) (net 4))
 (segment (start 90.97 114.95) (end 90.75 115.17) (width 0.4) (layer B.Cu) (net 4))
 (segment (start 92.5 112) (end 91.1 112) (width 0.4) (layer B.Cu) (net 4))
 (segment (start 91.1 112) (end 90.97 112.13) (width 0.4) (layer B.Cu) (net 4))
 (segment (start 86.04 121.54) (end 86.04 120.39) (width 0.4) (layer B.Cu) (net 4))
 (segment (start 86.04 120.39) (end 87.74 118.69) (width 0.4) (layer B.Cu) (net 4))
 (segment (start 84.1 122.25) (end 85.33 122.25) (width 0.4) (layer B.Cu) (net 4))
 (segment (start 85.33 122.25) (end 86.04 121.54) (width 0.4) (layer B.Cu) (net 4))
 (via (at 103.39 116.49) (size 0.6) (drill 0.4) (layers F.Cu B.Cu) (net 5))
 (segment (start 104 114.5) (end 103.12 115.38) (width 0.4) (layer B.Cu) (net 5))
 (segment (start 103.12 116.22) (end 103.12 115.38) (width 0.4) (layer B.Cu) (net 5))
 (segment (start 103.12 116.22) (end 103.39 116.49) (width 0.4) (layer B.Cu) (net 5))
 (segment (start 104 114.5) (end 104 112.99) (width 0.4) (layer B.Cu) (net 5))
 (segment (start 103.01 112) (end 96.5 112) (width 0.4) (layer B.Cu) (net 5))
 (segment (start 104 112.99) (end 103.01 112) (width 0.4) (layer B.Cu) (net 5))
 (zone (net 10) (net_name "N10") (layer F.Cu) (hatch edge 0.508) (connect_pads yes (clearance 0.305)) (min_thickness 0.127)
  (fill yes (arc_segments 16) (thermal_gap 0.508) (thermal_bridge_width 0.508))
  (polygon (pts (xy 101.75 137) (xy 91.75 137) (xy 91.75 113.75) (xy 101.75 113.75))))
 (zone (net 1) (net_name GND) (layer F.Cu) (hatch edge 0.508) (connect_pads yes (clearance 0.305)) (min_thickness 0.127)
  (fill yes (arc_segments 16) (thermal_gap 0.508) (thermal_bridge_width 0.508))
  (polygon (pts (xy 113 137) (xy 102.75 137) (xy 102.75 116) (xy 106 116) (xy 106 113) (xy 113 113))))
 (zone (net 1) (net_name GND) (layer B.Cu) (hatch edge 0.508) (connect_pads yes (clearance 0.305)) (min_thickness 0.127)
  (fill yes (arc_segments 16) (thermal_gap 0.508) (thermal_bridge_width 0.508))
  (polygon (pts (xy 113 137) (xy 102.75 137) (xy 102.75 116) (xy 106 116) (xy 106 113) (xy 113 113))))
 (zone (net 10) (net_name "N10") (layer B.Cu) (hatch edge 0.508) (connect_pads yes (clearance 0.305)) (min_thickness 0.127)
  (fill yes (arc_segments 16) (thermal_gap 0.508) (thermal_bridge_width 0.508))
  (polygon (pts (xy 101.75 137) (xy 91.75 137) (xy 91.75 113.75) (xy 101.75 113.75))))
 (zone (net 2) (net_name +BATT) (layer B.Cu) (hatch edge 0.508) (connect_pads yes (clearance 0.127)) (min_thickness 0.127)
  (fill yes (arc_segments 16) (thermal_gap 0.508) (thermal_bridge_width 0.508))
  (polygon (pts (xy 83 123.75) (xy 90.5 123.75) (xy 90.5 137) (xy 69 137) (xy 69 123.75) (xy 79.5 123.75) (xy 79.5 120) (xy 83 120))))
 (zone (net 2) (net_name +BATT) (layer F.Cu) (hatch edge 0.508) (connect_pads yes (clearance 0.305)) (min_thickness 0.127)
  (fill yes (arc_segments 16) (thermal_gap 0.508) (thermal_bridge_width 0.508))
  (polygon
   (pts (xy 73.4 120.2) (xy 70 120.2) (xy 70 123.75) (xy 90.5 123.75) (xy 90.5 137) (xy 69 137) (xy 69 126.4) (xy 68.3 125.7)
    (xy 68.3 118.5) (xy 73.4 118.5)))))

